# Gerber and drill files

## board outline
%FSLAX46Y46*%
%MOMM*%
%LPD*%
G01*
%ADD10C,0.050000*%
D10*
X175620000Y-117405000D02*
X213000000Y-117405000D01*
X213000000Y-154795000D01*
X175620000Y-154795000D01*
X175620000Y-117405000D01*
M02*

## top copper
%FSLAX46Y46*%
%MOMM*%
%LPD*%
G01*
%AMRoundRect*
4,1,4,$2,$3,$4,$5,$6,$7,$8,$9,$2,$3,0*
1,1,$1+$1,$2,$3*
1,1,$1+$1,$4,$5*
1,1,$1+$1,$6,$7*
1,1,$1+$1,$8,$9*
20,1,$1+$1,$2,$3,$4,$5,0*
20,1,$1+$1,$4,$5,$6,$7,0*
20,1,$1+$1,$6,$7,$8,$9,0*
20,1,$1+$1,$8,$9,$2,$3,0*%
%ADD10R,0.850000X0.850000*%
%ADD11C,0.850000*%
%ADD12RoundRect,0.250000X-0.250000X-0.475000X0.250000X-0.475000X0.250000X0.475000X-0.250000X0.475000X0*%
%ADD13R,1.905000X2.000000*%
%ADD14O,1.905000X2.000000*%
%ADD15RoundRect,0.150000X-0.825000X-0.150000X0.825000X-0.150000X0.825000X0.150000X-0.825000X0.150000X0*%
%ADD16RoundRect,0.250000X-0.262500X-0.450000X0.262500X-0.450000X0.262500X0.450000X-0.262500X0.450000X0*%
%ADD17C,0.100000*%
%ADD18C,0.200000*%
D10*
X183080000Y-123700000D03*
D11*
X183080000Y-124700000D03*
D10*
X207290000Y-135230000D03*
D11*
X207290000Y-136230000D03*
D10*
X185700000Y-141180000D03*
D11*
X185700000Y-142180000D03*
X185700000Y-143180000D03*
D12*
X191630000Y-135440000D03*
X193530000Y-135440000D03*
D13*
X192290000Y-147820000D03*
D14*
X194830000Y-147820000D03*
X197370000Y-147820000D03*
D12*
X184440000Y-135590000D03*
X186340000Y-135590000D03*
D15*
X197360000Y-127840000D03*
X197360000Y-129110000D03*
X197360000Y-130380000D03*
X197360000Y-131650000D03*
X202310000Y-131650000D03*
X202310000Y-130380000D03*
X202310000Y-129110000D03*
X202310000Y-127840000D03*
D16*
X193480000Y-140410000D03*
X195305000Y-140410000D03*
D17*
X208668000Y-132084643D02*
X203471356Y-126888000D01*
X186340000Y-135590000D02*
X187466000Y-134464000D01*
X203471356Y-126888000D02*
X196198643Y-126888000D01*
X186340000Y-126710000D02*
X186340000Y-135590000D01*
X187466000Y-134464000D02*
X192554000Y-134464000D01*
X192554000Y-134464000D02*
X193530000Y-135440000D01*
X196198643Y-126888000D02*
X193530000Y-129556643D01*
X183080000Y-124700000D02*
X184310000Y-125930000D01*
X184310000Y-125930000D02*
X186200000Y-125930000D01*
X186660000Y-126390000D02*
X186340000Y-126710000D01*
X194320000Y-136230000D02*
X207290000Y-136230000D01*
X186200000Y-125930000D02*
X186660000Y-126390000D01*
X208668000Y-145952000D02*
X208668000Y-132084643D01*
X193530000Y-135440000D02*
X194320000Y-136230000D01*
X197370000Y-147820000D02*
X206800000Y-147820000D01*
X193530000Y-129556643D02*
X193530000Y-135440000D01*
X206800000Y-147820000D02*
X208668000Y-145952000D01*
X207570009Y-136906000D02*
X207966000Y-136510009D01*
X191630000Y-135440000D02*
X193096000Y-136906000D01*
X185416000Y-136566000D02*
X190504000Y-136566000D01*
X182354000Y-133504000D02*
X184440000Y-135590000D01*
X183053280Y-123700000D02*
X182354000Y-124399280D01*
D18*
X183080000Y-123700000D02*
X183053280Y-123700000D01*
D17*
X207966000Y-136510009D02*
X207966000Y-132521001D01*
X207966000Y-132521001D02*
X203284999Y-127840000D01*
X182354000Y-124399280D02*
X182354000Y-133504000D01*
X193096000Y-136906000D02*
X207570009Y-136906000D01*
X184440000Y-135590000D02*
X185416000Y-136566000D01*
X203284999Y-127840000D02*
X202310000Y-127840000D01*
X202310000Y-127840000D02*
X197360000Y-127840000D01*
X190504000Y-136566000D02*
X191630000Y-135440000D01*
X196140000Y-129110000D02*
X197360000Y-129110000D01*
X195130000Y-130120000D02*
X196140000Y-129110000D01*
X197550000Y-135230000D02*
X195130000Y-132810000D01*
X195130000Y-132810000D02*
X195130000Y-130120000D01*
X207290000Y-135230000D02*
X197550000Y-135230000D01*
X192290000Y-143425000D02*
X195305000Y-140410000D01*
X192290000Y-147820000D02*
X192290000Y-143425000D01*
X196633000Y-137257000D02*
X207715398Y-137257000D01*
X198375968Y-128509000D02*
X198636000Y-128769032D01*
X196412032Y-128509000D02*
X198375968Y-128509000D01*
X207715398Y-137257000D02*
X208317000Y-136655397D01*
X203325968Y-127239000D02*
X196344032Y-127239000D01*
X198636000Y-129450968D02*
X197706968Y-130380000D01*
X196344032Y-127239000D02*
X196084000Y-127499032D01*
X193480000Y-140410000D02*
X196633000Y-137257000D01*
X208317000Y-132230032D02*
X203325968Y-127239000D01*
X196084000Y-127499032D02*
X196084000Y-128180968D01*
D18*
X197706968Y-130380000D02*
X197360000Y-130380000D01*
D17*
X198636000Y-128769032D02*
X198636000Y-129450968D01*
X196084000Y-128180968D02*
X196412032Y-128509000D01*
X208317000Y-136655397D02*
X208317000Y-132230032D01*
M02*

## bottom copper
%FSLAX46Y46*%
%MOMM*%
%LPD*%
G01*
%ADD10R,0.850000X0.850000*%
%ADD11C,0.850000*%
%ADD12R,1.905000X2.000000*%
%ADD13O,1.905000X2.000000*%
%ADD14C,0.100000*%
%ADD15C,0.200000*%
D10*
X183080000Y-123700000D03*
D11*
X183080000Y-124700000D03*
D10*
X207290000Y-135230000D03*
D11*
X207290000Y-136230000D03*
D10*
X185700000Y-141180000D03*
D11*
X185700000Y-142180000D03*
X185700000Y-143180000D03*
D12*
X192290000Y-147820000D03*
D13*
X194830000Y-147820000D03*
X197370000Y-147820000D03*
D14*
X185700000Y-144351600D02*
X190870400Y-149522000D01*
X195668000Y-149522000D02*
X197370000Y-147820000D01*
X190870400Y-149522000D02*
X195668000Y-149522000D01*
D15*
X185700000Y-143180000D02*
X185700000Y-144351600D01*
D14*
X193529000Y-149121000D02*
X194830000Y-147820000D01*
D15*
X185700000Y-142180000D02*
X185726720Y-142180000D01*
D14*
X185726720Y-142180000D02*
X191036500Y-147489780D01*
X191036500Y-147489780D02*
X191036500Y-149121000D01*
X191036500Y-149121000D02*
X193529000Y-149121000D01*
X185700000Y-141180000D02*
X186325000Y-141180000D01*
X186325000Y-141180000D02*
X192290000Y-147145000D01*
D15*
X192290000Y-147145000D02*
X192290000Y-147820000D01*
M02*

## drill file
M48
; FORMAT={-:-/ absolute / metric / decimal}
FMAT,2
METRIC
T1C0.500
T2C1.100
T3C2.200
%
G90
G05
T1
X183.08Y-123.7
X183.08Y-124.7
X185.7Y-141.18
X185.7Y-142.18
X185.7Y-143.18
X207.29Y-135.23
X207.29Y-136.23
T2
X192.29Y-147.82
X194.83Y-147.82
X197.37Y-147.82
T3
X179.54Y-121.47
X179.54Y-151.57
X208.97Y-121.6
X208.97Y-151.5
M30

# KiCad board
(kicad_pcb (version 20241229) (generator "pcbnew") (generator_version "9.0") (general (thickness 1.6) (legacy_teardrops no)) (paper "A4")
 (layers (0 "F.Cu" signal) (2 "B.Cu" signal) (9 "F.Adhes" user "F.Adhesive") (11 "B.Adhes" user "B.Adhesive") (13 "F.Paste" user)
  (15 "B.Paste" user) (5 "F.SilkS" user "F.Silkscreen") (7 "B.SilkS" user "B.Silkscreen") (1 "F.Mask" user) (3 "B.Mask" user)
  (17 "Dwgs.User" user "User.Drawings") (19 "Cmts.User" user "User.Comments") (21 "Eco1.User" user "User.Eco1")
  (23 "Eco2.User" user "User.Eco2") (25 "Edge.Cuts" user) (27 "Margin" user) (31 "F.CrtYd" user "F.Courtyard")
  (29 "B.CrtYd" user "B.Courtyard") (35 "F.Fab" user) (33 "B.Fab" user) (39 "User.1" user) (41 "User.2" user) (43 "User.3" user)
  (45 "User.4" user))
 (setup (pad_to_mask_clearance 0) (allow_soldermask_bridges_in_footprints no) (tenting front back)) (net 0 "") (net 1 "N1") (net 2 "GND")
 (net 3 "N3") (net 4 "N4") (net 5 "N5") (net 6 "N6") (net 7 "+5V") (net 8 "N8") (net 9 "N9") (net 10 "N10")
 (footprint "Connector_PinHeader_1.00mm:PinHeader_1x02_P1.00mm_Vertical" (layer "F.Cu") (at 183.08 123.7)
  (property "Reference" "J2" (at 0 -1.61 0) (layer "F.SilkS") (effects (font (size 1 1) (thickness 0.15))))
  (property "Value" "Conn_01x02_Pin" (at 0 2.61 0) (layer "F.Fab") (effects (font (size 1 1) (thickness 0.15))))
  (pad "1" thru_hole rect (at 0 0) (size 0.85 0.85) (drill 0.5) (layers "*.Cu" "*.Mask") (remove_unused_layers no) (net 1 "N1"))
  (pad "2" thru_hole circle (at 0 1) (size 0.85 0.85) (drill 0.5) (layers "*.Cu" "*.Mask") (remove_unused_layers no) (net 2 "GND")))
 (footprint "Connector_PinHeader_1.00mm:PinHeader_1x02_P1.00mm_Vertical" (layer "F.Cu") (at 207.29 135.23)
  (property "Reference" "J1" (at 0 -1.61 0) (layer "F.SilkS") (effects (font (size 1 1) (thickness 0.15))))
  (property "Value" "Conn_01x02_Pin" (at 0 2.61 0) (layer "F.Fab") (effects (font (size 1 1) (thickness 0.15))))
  (pad "1" thru_hole rect (at 0 0) (size 0.85 0.85) (drill 0.5) (layers "*.Cu" "*.Mask") (remove_unused_layers no) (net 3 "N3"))
  (pad "2" thru_hole circle (at 0 1) (size 0.85 0.85) (drill 0.5) (layers "*.Cu" "*.Mask") (remove_unused_layers no) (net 2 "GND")))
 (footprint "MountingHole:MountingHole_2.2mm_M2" (layer "F.Cu") (at 208.97 121.6)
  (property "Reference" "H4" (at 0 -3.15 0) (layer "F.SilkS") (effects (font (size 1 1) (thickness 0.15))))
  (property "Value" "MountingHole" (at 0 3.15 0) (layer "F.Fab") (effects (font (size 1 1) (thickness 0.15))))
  (pad "" np_thru_hole circle (at 0 0) (size 2.2 2.2) (drill 2.2) (layers "*.Cu" "*.Mask")))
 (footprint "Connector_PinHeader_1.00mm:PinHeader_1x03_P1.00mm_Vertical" (layer "F.Cu") (at 185.7 141.18)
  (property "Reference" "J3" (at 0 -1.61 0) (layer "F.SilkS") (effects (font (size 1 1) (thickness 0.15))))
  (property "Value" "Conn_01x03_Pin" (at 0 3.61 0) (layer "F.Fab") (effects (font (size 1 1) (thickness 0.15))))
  (pad "1" thru_hole rect (at 0 0) (size 0.85 0.85) (drill 0.5) (layers "*.Cu" "*.Mask") (remove_unused_layers no) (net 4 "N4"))
  (pad "2" thru_hole circle (at 0 1) (size 0.85 0.85) (drill 0.5) (layers "*.Cu" "*.Mask") (remove_unused_layers no) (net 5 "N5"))
  (pad "3" thru_hole circle (at 0 2) (size 0.85 0.85) (drill 0.5) (layers "*.Cu" "*.Mask") (remove_unused_layers no) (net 2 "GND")))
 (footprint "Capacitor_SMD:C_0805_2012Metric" (layer "F.Cu") (at 192.58 135.44)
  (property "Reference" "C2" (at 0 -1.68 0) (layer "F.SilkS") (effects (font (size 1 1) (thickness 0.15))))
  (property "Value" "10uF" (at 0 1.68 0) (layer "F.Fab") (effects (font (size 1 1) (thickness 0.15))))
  (pad "1" smd roundrect (at -0.95 0) (size 1 1.45) (layers "F.Cu" "F.Mask" "F.Paste") (roundrect_rratio 0.25) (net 1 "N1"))
  (pad "2" smd roundrect (at 0.95 0) (size 1 1.45) (layers "F.Cu" "F.Mask" "F.Paste") (roundrect_rratio 0.25) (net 2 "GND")))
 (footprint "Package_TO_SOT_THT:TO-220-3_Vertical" (layer "F.Cu") (at 192.29 147.82)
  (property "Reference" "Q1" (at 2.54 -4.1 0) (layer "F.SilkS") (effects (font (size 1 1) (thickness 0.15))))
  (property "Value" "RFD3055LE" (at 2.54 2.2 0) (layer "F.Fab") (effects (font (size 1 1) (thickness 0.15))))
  (pad "1" thru_hole rect (at 0 0) (size 1.905 2) (drill 1.1) (layers "*.Cu" "*.Mask") (remove_unused_layers no) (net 4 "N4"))
  (pad "2" thru_hole oval (at 2.54 0) (size 1.905 2) (drill 1.1) (layers "*.Cu" "*.Mask") (remove_unused_layers no) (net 5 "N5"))
  (pad "3" thru_hole oval (at 5.08 0) (size 1.905 2) (drill 1.1) (layers "*.Cu" "*.Mask") (remove_unused_layers no) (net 2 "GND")))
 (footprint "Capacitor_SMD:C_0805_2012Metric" (layer "F.Cu") (at 185.39 135.59)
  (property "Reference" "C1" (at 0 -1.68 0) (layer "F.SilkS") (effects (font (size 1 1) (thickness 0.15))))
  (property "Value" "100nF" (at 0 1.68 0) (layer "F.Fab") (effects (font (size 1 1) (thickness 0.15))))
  (pad "1" smd roundrect (at -0.95 0) (size 1 1.45) (layers "F.Cu" "F.Mask" "F.Paste") (roundrect_rratio 0.25) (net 1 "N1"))
  (pad "2" smd roundrect (at 0.95 0) (size 1 1.45) (layers "F.Cu" "F.Mask" "F.Paste") (roundrect_rratio 0.25) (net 2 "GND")))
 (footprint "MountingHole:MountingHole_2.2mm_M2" (layer "F.Cu") (at 179.54 151.57)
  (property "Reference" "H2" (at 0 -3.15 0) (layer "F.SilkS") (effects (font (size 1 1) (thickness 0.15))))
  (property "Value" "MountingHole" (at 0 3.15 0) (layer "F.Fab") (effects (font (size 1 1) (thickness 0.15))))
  (pad "" np_thru_hole circle (at 0 0) (size 2.2 2.2) (drill 2.2) (layers "*.Cu" "*.Mask")))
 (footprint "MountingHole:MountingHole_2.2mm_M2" (layer "F.Cu") (at 208.97 151.5)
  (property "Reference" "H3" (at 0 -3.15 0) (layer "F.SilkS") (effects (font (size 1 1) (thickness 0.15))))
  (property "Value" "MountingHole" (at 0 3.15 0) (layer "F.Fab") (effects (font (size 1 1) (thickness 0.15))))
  (pad "" np_thru_hole circle (at 0 0) (size 2.2 2.2) (drill 2.2) (layers "*.Cu" "*.Mask")))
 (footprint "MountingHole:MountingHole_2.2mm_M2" (layer "F.Cu") (at 179.54 121.47)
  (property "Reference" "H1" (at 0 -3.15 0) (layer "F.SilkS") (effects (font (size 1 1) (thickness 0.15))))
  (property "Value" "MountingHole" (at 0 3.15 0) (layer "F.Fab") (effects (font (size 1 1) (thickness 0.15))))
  (pad "" np_thru_hole circle (at 0 0) (size 2.2 2.2) (drill 2.2) (layers "*.Cu" "*.Mask")))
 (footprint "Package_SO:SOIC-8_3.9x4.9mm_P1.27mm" (layer "F.Cu") (at 199.835 129.745)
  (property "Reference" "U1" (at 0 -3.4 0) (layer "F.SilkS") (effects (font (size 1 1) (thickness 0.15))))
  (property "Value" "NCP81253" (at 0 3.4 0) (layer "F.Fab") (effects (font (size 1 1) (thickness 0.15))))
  (pad "1" smd roundrect (at -2.475 -1.905) (size 1.95 0.6) (layers "F.Cu" "F.Mask" "F.Paste") (roundrect_rratio 0.25) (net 1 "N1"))
  (pad "2" smd roundrect (at -2.475 -0.635) (size 1.95 0.6) (layers "F.Cu" "F.Mask" "F.Paste") (roundrect_rratio 0.25) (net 3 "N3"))
  (pad "3" smd roundrect (at -2.475 0.635) (size 1.95 0.6) (layers "F.Cu" "F.Mask" "F.Paste") (roundrect_rratio 0.25) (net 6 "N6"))
  (pad "4" smd roundrect (at -2.475 1.905) (size 1.95 0.6) (layers "F.Cu" "F.Mask" "F.Paste") (roundrect_rratio 0.25) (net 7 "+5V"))
  (pad "5" smd roundrect (at 2.475 1.905) (size 1.95 0.6) (layers "F.Cu" "F.Mask" "F.Paste") (roundrect_rratio 0.25) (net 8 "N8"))
  (pad "6" smd roundrect (at 2.475 0.635) (size 1.95 0.6) (layers "F.Cu" "F.Mask" "F.Paste") (roundrect_rratio 0.25) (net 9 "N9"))
  (pad "7" smd roundrect (at 2.475 -0.635) (size 1.95 0.6) (layers "F.Cu" "F.Mask" "F.Paste") (roundrect_rratio 0.25) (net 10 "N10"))
  (pad "8" smd roundrect (at 2.475 -1.905) (size 1.95 0.6) (layers "F.Cu" "F.Mask" "F.Paste") (roundrect_rratio 0.25) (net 1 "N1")))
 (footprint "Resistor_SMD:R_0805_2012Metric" (layer "F.Cu") (at 194.3925 140.41)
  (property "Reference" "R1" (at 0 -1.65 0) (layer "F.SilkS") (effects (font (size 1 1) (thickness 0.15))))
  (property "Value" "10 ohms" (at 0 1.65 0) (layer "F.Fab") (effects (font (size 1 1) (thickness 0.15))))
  (pad "1" smd roundrect (at -0.9125 0) (size 1.025 1.4) (layers "F.Cu" "F.Mask" "F.Paste") (roundrect_rratio 0.243902) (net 6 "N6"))
  (pad "2" smd roundrect (at 0.9125 0) (size 1.025 1.4) (layers "F.Cu" "F.Mask" "F.Paste") (roundrect_rratio 0.243902) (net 4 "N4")))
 (gr_rect (start 175.62 117.405) (end 213 154.795) (stroke (width 0.05) (type default)) (fill no) (layer "Edge.Cuts"))
 (segment (start 208.668 132.084643) (end 203.471356 126.888) (width 0.1) (layer "F.Cu") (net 2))
 (segment (start 186.34 135.59) (end 187.466 134.464) (width 0.1) (layer "F.Cu") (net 2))
 (segment (start 203.471356 126.888) (end 196.198643 126.888) (width 0.1) (layer "F.Cu") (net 2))
 (segment (start 186.34 126.71) (end 186.34 135.59) (width 0.1) (layer "F.Cu") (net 2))
 (segment (start 187.466 134.464) (end 192.554 134.464) (width 0.1) (layer "F.Cu") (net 2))
 (segment (start 192.554 134.464) (end 193.53 135.44) (width 0.1) (layer "F.Cu") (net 2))
 (segment (start 196.198643 126.888) (end 193.53 129.556643) (width 0.1) (layer "F.Cu") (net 2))
 (segment (start 183.08 124.7) (end 184.31 125.93) (width 0.1) (layer "F.Cu") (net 2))
 (segment (start 184.31 125.93) (end 186.2 125.93) (width 0.1) (layer "F.Cu") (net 2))
 (segment (start 186.66 126.39) (end 186.34 126.71) (width 0.1) (layer "F.Cu") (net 2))
 (segment (start 194.32 136.23) (end 207.29 136.23) (width 0.1) (layer "F.Cu") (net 2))
 (segment (start 186.2 125.93) (end 186.66 126.39) (width 0.1) (layer "F.Cu") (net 2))
 (segment (start 208.668 145.952) (end 208.668 132.084643) (width 0.1) (layer "F.Cu") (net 2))
 (segment (start 193.53 135.44) (end 194.32 136.23) (width 0.1) (layer "F.Cu") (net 2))
 (segment (start 197.37 147.82) (end 206.8 147.82) (width 0.1) (layer "F.Cu") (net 2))
 (segment (start 193.53 129.556643) (end 193.53 135.44) (width 0.1) (layer "F.Cu") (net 2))
 (segment (start 206.8 147.82) (end 208.668 145.952) (width 0.1) (layer "F.Cu") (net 2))
 (segment (start 185.7 144.3516) (end 190.8704 149.522) (width 0.1) (layer "B.Cu") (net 2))
 (segment (start 195.668 149.522) (end 197.37 147.82) (width 0.1) (layer "B.Cu") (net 2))
 (segment (start 190.8704 149.522) (end 195.668 149.522) (width 0.1) (layer "B.Cu") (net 2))
 (segment (start 185.7 143.18) (end 185.7 144.3516) (width 0.2) (layer "B.Cu") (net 2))
 (segment (start 207.570009 136.906) (end 207.966 136.510009) (width 0.1) (layer "F.Cu") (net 1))
 (segment (start 191.63 135.44) (end 193.096 136.906) (width 0.1) (layer "F.Cu") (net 1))
 (segment (start 185.416 136.566) (end 190.504 136.566) (width 0.1) (layer "F.Cu") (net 1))
 (segment (start 182.354 133.504) (end 184.44 135.59) (width 0.1) (layer "F.Cu") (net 1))
 (segment (start 183.05328 123.7) (end 182.354 124.39928) (width 0.1) (layer "F.Cu") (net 1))
 (segment (start 183.08 123.7) (end 183.05328 123.7) (width 0.2) (layer "F.Cu") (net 1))
 (segment (start 207.966 136.510009) (end 207.966 132.521001) (width 0.1) (layer "F.Cu") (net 1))
 (segment (start 207.966 132.521001) (end 203.284999 127.84) (width 0.1) (layer "F.Cu") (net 1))
 (segment (start 182.354 124.39928) (end 182.354 133.504) (width 0.1) (layer "F.Cu") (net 1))
 (segment (start 193.096 136.906) (end 207.570009 136.906) (width 0.1) (layer "F.Cu") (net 1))
 (segment (start 184.44 135.59) (end 185.416 136.566) (width 0.1) (layer "F.Cu") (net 1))
 (segment (start 203.284999 127.84) (end 202.31 127.84) (width 0.1) (layer "F.Cu") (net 1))
 (segment (start 202.31 127.84) (end 197.36 127.84) (width 0.1) (layer "F.Cu") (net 1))
 (segment (start 190.504 136.566) (end 191.63 135.44) (width 0.1) (layer "F.Cu") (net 1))
 (segment (start 196.14 129.11) (end 197.36 129.11) (width 0.1) (layer "F.Cu") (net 3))
 (segment (start 195.13 130.12) (end 196.14 129.11) (width 0.1) (layer "F.Cu") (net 3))
 (segment (start 197.55 135.23) (end 195.13 132.81) (width 0.1) (layer "F.Cu") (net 3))
 (segment (start 195.13 132.81) (end 195.13 130.12) (width 0.1) (layer "F.Cu") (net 3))
 (segment (start 207.29 135.23) (end 197.55 135.23) (width 0.1) (layer "F.Cu") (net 3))
 (segment (start 193.529 149.121) (end 194.83 147.82) (width 0.1) (layer "B.Cu") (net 5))
 (segment (start 185.7 142.18) (end 185.72672 142.18) (width 0.2) (layer "B.Cu") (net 5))
 (segment (start 185.72672 142.18) (end 191.0365 147.48978) (width 0.1) (layer "B.Cu") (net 5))
 (segment (start 191.0365 147.48978) (end 191.0365 149.121) (width 0.1) (layer "B.Cu") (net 5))
 (segment (start 191.0365 149.121) (end 193.529 149.121) (width 0.1) (layer "B.Cu") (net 5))
 (segment (start 192.29 143.425) (end 195.305 140.41) (width 0.1) (layer "F.Cu") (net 4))
 (segment (start 192.29 147.82) (end 192.29 143.425) (width 0.1) (layer "F.Cu") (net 4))
 (segment (start 185.7 141.18) (end 186.325 141.18) (width 0.1) (layer "B.Cu") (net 4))
 (segment (start 186.325 141.18) (end 192.29 147.145) (width 0.1) (layer "B.Cu") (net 4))
 (segment (start 192.29 147.145) (end 192.29 147.82) (width 0.2) (layer "B.Cu") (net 4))
 (segment (start 196.633 137.257) (end 207.715398 137.257) (width 0.1) (layer "F.Cu") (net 6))
 (segment (start 198.375968 128.509) (end 198.636 128.769032) (width 0.1) (layer "F.Cu") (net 6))
 (segment (start 196.412032 128.509) (end 198.375968 128.509) (width 0.1) (layer "F.Cu") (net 6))
 (segment (start 207.715398 137.257) (end 208.317 136.655397) (width 0.1) (layer "F.Cu") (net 6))
 (segment (start 203.325968 127.239) (end 196.344032 127.239) (width 0.1) (layer "F.Cu") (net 6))
 (segment (start 198.636 129.450968) (end 197.706968 130.38) (width 0.1) (layer "F.Cu") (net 6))
 (segment (start 196.344032 127.239) (end 196.084 127.499032) (width 0.1) (layer "F.Cu") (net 6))
 (segment (start 193.48 140.41) (end 196.633 137.257) (width 0.1) (layer "F.Cu") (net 6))
 (segment (start 208.317 132.230032) (end 203.325968 127.239) (width 0.1) (layer "F.Cu") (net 6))
 (segment (start 196.084 127.499032) (end 196.084 128.180968) (width 0.1) (layer "F.Cu") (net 6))
 (segment (start 197.706968 130.38) (end 197.36 130.38) (width 0.2) (layer "F.Cu") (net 6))
 (segment (start 198.636 128.769032) (end 198.636 129.450968) (width 0.1) (layer "F.Cu") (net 6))
 (segment (start 196.084 128.180968) (end 196.412032 128.509) (width 0.1) (layer "F.Cu") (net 6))
 (segment (start 208.317 136.655397) (end 208.317 132.230032) (width 0.1) (layer "F.Cu") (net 6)))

